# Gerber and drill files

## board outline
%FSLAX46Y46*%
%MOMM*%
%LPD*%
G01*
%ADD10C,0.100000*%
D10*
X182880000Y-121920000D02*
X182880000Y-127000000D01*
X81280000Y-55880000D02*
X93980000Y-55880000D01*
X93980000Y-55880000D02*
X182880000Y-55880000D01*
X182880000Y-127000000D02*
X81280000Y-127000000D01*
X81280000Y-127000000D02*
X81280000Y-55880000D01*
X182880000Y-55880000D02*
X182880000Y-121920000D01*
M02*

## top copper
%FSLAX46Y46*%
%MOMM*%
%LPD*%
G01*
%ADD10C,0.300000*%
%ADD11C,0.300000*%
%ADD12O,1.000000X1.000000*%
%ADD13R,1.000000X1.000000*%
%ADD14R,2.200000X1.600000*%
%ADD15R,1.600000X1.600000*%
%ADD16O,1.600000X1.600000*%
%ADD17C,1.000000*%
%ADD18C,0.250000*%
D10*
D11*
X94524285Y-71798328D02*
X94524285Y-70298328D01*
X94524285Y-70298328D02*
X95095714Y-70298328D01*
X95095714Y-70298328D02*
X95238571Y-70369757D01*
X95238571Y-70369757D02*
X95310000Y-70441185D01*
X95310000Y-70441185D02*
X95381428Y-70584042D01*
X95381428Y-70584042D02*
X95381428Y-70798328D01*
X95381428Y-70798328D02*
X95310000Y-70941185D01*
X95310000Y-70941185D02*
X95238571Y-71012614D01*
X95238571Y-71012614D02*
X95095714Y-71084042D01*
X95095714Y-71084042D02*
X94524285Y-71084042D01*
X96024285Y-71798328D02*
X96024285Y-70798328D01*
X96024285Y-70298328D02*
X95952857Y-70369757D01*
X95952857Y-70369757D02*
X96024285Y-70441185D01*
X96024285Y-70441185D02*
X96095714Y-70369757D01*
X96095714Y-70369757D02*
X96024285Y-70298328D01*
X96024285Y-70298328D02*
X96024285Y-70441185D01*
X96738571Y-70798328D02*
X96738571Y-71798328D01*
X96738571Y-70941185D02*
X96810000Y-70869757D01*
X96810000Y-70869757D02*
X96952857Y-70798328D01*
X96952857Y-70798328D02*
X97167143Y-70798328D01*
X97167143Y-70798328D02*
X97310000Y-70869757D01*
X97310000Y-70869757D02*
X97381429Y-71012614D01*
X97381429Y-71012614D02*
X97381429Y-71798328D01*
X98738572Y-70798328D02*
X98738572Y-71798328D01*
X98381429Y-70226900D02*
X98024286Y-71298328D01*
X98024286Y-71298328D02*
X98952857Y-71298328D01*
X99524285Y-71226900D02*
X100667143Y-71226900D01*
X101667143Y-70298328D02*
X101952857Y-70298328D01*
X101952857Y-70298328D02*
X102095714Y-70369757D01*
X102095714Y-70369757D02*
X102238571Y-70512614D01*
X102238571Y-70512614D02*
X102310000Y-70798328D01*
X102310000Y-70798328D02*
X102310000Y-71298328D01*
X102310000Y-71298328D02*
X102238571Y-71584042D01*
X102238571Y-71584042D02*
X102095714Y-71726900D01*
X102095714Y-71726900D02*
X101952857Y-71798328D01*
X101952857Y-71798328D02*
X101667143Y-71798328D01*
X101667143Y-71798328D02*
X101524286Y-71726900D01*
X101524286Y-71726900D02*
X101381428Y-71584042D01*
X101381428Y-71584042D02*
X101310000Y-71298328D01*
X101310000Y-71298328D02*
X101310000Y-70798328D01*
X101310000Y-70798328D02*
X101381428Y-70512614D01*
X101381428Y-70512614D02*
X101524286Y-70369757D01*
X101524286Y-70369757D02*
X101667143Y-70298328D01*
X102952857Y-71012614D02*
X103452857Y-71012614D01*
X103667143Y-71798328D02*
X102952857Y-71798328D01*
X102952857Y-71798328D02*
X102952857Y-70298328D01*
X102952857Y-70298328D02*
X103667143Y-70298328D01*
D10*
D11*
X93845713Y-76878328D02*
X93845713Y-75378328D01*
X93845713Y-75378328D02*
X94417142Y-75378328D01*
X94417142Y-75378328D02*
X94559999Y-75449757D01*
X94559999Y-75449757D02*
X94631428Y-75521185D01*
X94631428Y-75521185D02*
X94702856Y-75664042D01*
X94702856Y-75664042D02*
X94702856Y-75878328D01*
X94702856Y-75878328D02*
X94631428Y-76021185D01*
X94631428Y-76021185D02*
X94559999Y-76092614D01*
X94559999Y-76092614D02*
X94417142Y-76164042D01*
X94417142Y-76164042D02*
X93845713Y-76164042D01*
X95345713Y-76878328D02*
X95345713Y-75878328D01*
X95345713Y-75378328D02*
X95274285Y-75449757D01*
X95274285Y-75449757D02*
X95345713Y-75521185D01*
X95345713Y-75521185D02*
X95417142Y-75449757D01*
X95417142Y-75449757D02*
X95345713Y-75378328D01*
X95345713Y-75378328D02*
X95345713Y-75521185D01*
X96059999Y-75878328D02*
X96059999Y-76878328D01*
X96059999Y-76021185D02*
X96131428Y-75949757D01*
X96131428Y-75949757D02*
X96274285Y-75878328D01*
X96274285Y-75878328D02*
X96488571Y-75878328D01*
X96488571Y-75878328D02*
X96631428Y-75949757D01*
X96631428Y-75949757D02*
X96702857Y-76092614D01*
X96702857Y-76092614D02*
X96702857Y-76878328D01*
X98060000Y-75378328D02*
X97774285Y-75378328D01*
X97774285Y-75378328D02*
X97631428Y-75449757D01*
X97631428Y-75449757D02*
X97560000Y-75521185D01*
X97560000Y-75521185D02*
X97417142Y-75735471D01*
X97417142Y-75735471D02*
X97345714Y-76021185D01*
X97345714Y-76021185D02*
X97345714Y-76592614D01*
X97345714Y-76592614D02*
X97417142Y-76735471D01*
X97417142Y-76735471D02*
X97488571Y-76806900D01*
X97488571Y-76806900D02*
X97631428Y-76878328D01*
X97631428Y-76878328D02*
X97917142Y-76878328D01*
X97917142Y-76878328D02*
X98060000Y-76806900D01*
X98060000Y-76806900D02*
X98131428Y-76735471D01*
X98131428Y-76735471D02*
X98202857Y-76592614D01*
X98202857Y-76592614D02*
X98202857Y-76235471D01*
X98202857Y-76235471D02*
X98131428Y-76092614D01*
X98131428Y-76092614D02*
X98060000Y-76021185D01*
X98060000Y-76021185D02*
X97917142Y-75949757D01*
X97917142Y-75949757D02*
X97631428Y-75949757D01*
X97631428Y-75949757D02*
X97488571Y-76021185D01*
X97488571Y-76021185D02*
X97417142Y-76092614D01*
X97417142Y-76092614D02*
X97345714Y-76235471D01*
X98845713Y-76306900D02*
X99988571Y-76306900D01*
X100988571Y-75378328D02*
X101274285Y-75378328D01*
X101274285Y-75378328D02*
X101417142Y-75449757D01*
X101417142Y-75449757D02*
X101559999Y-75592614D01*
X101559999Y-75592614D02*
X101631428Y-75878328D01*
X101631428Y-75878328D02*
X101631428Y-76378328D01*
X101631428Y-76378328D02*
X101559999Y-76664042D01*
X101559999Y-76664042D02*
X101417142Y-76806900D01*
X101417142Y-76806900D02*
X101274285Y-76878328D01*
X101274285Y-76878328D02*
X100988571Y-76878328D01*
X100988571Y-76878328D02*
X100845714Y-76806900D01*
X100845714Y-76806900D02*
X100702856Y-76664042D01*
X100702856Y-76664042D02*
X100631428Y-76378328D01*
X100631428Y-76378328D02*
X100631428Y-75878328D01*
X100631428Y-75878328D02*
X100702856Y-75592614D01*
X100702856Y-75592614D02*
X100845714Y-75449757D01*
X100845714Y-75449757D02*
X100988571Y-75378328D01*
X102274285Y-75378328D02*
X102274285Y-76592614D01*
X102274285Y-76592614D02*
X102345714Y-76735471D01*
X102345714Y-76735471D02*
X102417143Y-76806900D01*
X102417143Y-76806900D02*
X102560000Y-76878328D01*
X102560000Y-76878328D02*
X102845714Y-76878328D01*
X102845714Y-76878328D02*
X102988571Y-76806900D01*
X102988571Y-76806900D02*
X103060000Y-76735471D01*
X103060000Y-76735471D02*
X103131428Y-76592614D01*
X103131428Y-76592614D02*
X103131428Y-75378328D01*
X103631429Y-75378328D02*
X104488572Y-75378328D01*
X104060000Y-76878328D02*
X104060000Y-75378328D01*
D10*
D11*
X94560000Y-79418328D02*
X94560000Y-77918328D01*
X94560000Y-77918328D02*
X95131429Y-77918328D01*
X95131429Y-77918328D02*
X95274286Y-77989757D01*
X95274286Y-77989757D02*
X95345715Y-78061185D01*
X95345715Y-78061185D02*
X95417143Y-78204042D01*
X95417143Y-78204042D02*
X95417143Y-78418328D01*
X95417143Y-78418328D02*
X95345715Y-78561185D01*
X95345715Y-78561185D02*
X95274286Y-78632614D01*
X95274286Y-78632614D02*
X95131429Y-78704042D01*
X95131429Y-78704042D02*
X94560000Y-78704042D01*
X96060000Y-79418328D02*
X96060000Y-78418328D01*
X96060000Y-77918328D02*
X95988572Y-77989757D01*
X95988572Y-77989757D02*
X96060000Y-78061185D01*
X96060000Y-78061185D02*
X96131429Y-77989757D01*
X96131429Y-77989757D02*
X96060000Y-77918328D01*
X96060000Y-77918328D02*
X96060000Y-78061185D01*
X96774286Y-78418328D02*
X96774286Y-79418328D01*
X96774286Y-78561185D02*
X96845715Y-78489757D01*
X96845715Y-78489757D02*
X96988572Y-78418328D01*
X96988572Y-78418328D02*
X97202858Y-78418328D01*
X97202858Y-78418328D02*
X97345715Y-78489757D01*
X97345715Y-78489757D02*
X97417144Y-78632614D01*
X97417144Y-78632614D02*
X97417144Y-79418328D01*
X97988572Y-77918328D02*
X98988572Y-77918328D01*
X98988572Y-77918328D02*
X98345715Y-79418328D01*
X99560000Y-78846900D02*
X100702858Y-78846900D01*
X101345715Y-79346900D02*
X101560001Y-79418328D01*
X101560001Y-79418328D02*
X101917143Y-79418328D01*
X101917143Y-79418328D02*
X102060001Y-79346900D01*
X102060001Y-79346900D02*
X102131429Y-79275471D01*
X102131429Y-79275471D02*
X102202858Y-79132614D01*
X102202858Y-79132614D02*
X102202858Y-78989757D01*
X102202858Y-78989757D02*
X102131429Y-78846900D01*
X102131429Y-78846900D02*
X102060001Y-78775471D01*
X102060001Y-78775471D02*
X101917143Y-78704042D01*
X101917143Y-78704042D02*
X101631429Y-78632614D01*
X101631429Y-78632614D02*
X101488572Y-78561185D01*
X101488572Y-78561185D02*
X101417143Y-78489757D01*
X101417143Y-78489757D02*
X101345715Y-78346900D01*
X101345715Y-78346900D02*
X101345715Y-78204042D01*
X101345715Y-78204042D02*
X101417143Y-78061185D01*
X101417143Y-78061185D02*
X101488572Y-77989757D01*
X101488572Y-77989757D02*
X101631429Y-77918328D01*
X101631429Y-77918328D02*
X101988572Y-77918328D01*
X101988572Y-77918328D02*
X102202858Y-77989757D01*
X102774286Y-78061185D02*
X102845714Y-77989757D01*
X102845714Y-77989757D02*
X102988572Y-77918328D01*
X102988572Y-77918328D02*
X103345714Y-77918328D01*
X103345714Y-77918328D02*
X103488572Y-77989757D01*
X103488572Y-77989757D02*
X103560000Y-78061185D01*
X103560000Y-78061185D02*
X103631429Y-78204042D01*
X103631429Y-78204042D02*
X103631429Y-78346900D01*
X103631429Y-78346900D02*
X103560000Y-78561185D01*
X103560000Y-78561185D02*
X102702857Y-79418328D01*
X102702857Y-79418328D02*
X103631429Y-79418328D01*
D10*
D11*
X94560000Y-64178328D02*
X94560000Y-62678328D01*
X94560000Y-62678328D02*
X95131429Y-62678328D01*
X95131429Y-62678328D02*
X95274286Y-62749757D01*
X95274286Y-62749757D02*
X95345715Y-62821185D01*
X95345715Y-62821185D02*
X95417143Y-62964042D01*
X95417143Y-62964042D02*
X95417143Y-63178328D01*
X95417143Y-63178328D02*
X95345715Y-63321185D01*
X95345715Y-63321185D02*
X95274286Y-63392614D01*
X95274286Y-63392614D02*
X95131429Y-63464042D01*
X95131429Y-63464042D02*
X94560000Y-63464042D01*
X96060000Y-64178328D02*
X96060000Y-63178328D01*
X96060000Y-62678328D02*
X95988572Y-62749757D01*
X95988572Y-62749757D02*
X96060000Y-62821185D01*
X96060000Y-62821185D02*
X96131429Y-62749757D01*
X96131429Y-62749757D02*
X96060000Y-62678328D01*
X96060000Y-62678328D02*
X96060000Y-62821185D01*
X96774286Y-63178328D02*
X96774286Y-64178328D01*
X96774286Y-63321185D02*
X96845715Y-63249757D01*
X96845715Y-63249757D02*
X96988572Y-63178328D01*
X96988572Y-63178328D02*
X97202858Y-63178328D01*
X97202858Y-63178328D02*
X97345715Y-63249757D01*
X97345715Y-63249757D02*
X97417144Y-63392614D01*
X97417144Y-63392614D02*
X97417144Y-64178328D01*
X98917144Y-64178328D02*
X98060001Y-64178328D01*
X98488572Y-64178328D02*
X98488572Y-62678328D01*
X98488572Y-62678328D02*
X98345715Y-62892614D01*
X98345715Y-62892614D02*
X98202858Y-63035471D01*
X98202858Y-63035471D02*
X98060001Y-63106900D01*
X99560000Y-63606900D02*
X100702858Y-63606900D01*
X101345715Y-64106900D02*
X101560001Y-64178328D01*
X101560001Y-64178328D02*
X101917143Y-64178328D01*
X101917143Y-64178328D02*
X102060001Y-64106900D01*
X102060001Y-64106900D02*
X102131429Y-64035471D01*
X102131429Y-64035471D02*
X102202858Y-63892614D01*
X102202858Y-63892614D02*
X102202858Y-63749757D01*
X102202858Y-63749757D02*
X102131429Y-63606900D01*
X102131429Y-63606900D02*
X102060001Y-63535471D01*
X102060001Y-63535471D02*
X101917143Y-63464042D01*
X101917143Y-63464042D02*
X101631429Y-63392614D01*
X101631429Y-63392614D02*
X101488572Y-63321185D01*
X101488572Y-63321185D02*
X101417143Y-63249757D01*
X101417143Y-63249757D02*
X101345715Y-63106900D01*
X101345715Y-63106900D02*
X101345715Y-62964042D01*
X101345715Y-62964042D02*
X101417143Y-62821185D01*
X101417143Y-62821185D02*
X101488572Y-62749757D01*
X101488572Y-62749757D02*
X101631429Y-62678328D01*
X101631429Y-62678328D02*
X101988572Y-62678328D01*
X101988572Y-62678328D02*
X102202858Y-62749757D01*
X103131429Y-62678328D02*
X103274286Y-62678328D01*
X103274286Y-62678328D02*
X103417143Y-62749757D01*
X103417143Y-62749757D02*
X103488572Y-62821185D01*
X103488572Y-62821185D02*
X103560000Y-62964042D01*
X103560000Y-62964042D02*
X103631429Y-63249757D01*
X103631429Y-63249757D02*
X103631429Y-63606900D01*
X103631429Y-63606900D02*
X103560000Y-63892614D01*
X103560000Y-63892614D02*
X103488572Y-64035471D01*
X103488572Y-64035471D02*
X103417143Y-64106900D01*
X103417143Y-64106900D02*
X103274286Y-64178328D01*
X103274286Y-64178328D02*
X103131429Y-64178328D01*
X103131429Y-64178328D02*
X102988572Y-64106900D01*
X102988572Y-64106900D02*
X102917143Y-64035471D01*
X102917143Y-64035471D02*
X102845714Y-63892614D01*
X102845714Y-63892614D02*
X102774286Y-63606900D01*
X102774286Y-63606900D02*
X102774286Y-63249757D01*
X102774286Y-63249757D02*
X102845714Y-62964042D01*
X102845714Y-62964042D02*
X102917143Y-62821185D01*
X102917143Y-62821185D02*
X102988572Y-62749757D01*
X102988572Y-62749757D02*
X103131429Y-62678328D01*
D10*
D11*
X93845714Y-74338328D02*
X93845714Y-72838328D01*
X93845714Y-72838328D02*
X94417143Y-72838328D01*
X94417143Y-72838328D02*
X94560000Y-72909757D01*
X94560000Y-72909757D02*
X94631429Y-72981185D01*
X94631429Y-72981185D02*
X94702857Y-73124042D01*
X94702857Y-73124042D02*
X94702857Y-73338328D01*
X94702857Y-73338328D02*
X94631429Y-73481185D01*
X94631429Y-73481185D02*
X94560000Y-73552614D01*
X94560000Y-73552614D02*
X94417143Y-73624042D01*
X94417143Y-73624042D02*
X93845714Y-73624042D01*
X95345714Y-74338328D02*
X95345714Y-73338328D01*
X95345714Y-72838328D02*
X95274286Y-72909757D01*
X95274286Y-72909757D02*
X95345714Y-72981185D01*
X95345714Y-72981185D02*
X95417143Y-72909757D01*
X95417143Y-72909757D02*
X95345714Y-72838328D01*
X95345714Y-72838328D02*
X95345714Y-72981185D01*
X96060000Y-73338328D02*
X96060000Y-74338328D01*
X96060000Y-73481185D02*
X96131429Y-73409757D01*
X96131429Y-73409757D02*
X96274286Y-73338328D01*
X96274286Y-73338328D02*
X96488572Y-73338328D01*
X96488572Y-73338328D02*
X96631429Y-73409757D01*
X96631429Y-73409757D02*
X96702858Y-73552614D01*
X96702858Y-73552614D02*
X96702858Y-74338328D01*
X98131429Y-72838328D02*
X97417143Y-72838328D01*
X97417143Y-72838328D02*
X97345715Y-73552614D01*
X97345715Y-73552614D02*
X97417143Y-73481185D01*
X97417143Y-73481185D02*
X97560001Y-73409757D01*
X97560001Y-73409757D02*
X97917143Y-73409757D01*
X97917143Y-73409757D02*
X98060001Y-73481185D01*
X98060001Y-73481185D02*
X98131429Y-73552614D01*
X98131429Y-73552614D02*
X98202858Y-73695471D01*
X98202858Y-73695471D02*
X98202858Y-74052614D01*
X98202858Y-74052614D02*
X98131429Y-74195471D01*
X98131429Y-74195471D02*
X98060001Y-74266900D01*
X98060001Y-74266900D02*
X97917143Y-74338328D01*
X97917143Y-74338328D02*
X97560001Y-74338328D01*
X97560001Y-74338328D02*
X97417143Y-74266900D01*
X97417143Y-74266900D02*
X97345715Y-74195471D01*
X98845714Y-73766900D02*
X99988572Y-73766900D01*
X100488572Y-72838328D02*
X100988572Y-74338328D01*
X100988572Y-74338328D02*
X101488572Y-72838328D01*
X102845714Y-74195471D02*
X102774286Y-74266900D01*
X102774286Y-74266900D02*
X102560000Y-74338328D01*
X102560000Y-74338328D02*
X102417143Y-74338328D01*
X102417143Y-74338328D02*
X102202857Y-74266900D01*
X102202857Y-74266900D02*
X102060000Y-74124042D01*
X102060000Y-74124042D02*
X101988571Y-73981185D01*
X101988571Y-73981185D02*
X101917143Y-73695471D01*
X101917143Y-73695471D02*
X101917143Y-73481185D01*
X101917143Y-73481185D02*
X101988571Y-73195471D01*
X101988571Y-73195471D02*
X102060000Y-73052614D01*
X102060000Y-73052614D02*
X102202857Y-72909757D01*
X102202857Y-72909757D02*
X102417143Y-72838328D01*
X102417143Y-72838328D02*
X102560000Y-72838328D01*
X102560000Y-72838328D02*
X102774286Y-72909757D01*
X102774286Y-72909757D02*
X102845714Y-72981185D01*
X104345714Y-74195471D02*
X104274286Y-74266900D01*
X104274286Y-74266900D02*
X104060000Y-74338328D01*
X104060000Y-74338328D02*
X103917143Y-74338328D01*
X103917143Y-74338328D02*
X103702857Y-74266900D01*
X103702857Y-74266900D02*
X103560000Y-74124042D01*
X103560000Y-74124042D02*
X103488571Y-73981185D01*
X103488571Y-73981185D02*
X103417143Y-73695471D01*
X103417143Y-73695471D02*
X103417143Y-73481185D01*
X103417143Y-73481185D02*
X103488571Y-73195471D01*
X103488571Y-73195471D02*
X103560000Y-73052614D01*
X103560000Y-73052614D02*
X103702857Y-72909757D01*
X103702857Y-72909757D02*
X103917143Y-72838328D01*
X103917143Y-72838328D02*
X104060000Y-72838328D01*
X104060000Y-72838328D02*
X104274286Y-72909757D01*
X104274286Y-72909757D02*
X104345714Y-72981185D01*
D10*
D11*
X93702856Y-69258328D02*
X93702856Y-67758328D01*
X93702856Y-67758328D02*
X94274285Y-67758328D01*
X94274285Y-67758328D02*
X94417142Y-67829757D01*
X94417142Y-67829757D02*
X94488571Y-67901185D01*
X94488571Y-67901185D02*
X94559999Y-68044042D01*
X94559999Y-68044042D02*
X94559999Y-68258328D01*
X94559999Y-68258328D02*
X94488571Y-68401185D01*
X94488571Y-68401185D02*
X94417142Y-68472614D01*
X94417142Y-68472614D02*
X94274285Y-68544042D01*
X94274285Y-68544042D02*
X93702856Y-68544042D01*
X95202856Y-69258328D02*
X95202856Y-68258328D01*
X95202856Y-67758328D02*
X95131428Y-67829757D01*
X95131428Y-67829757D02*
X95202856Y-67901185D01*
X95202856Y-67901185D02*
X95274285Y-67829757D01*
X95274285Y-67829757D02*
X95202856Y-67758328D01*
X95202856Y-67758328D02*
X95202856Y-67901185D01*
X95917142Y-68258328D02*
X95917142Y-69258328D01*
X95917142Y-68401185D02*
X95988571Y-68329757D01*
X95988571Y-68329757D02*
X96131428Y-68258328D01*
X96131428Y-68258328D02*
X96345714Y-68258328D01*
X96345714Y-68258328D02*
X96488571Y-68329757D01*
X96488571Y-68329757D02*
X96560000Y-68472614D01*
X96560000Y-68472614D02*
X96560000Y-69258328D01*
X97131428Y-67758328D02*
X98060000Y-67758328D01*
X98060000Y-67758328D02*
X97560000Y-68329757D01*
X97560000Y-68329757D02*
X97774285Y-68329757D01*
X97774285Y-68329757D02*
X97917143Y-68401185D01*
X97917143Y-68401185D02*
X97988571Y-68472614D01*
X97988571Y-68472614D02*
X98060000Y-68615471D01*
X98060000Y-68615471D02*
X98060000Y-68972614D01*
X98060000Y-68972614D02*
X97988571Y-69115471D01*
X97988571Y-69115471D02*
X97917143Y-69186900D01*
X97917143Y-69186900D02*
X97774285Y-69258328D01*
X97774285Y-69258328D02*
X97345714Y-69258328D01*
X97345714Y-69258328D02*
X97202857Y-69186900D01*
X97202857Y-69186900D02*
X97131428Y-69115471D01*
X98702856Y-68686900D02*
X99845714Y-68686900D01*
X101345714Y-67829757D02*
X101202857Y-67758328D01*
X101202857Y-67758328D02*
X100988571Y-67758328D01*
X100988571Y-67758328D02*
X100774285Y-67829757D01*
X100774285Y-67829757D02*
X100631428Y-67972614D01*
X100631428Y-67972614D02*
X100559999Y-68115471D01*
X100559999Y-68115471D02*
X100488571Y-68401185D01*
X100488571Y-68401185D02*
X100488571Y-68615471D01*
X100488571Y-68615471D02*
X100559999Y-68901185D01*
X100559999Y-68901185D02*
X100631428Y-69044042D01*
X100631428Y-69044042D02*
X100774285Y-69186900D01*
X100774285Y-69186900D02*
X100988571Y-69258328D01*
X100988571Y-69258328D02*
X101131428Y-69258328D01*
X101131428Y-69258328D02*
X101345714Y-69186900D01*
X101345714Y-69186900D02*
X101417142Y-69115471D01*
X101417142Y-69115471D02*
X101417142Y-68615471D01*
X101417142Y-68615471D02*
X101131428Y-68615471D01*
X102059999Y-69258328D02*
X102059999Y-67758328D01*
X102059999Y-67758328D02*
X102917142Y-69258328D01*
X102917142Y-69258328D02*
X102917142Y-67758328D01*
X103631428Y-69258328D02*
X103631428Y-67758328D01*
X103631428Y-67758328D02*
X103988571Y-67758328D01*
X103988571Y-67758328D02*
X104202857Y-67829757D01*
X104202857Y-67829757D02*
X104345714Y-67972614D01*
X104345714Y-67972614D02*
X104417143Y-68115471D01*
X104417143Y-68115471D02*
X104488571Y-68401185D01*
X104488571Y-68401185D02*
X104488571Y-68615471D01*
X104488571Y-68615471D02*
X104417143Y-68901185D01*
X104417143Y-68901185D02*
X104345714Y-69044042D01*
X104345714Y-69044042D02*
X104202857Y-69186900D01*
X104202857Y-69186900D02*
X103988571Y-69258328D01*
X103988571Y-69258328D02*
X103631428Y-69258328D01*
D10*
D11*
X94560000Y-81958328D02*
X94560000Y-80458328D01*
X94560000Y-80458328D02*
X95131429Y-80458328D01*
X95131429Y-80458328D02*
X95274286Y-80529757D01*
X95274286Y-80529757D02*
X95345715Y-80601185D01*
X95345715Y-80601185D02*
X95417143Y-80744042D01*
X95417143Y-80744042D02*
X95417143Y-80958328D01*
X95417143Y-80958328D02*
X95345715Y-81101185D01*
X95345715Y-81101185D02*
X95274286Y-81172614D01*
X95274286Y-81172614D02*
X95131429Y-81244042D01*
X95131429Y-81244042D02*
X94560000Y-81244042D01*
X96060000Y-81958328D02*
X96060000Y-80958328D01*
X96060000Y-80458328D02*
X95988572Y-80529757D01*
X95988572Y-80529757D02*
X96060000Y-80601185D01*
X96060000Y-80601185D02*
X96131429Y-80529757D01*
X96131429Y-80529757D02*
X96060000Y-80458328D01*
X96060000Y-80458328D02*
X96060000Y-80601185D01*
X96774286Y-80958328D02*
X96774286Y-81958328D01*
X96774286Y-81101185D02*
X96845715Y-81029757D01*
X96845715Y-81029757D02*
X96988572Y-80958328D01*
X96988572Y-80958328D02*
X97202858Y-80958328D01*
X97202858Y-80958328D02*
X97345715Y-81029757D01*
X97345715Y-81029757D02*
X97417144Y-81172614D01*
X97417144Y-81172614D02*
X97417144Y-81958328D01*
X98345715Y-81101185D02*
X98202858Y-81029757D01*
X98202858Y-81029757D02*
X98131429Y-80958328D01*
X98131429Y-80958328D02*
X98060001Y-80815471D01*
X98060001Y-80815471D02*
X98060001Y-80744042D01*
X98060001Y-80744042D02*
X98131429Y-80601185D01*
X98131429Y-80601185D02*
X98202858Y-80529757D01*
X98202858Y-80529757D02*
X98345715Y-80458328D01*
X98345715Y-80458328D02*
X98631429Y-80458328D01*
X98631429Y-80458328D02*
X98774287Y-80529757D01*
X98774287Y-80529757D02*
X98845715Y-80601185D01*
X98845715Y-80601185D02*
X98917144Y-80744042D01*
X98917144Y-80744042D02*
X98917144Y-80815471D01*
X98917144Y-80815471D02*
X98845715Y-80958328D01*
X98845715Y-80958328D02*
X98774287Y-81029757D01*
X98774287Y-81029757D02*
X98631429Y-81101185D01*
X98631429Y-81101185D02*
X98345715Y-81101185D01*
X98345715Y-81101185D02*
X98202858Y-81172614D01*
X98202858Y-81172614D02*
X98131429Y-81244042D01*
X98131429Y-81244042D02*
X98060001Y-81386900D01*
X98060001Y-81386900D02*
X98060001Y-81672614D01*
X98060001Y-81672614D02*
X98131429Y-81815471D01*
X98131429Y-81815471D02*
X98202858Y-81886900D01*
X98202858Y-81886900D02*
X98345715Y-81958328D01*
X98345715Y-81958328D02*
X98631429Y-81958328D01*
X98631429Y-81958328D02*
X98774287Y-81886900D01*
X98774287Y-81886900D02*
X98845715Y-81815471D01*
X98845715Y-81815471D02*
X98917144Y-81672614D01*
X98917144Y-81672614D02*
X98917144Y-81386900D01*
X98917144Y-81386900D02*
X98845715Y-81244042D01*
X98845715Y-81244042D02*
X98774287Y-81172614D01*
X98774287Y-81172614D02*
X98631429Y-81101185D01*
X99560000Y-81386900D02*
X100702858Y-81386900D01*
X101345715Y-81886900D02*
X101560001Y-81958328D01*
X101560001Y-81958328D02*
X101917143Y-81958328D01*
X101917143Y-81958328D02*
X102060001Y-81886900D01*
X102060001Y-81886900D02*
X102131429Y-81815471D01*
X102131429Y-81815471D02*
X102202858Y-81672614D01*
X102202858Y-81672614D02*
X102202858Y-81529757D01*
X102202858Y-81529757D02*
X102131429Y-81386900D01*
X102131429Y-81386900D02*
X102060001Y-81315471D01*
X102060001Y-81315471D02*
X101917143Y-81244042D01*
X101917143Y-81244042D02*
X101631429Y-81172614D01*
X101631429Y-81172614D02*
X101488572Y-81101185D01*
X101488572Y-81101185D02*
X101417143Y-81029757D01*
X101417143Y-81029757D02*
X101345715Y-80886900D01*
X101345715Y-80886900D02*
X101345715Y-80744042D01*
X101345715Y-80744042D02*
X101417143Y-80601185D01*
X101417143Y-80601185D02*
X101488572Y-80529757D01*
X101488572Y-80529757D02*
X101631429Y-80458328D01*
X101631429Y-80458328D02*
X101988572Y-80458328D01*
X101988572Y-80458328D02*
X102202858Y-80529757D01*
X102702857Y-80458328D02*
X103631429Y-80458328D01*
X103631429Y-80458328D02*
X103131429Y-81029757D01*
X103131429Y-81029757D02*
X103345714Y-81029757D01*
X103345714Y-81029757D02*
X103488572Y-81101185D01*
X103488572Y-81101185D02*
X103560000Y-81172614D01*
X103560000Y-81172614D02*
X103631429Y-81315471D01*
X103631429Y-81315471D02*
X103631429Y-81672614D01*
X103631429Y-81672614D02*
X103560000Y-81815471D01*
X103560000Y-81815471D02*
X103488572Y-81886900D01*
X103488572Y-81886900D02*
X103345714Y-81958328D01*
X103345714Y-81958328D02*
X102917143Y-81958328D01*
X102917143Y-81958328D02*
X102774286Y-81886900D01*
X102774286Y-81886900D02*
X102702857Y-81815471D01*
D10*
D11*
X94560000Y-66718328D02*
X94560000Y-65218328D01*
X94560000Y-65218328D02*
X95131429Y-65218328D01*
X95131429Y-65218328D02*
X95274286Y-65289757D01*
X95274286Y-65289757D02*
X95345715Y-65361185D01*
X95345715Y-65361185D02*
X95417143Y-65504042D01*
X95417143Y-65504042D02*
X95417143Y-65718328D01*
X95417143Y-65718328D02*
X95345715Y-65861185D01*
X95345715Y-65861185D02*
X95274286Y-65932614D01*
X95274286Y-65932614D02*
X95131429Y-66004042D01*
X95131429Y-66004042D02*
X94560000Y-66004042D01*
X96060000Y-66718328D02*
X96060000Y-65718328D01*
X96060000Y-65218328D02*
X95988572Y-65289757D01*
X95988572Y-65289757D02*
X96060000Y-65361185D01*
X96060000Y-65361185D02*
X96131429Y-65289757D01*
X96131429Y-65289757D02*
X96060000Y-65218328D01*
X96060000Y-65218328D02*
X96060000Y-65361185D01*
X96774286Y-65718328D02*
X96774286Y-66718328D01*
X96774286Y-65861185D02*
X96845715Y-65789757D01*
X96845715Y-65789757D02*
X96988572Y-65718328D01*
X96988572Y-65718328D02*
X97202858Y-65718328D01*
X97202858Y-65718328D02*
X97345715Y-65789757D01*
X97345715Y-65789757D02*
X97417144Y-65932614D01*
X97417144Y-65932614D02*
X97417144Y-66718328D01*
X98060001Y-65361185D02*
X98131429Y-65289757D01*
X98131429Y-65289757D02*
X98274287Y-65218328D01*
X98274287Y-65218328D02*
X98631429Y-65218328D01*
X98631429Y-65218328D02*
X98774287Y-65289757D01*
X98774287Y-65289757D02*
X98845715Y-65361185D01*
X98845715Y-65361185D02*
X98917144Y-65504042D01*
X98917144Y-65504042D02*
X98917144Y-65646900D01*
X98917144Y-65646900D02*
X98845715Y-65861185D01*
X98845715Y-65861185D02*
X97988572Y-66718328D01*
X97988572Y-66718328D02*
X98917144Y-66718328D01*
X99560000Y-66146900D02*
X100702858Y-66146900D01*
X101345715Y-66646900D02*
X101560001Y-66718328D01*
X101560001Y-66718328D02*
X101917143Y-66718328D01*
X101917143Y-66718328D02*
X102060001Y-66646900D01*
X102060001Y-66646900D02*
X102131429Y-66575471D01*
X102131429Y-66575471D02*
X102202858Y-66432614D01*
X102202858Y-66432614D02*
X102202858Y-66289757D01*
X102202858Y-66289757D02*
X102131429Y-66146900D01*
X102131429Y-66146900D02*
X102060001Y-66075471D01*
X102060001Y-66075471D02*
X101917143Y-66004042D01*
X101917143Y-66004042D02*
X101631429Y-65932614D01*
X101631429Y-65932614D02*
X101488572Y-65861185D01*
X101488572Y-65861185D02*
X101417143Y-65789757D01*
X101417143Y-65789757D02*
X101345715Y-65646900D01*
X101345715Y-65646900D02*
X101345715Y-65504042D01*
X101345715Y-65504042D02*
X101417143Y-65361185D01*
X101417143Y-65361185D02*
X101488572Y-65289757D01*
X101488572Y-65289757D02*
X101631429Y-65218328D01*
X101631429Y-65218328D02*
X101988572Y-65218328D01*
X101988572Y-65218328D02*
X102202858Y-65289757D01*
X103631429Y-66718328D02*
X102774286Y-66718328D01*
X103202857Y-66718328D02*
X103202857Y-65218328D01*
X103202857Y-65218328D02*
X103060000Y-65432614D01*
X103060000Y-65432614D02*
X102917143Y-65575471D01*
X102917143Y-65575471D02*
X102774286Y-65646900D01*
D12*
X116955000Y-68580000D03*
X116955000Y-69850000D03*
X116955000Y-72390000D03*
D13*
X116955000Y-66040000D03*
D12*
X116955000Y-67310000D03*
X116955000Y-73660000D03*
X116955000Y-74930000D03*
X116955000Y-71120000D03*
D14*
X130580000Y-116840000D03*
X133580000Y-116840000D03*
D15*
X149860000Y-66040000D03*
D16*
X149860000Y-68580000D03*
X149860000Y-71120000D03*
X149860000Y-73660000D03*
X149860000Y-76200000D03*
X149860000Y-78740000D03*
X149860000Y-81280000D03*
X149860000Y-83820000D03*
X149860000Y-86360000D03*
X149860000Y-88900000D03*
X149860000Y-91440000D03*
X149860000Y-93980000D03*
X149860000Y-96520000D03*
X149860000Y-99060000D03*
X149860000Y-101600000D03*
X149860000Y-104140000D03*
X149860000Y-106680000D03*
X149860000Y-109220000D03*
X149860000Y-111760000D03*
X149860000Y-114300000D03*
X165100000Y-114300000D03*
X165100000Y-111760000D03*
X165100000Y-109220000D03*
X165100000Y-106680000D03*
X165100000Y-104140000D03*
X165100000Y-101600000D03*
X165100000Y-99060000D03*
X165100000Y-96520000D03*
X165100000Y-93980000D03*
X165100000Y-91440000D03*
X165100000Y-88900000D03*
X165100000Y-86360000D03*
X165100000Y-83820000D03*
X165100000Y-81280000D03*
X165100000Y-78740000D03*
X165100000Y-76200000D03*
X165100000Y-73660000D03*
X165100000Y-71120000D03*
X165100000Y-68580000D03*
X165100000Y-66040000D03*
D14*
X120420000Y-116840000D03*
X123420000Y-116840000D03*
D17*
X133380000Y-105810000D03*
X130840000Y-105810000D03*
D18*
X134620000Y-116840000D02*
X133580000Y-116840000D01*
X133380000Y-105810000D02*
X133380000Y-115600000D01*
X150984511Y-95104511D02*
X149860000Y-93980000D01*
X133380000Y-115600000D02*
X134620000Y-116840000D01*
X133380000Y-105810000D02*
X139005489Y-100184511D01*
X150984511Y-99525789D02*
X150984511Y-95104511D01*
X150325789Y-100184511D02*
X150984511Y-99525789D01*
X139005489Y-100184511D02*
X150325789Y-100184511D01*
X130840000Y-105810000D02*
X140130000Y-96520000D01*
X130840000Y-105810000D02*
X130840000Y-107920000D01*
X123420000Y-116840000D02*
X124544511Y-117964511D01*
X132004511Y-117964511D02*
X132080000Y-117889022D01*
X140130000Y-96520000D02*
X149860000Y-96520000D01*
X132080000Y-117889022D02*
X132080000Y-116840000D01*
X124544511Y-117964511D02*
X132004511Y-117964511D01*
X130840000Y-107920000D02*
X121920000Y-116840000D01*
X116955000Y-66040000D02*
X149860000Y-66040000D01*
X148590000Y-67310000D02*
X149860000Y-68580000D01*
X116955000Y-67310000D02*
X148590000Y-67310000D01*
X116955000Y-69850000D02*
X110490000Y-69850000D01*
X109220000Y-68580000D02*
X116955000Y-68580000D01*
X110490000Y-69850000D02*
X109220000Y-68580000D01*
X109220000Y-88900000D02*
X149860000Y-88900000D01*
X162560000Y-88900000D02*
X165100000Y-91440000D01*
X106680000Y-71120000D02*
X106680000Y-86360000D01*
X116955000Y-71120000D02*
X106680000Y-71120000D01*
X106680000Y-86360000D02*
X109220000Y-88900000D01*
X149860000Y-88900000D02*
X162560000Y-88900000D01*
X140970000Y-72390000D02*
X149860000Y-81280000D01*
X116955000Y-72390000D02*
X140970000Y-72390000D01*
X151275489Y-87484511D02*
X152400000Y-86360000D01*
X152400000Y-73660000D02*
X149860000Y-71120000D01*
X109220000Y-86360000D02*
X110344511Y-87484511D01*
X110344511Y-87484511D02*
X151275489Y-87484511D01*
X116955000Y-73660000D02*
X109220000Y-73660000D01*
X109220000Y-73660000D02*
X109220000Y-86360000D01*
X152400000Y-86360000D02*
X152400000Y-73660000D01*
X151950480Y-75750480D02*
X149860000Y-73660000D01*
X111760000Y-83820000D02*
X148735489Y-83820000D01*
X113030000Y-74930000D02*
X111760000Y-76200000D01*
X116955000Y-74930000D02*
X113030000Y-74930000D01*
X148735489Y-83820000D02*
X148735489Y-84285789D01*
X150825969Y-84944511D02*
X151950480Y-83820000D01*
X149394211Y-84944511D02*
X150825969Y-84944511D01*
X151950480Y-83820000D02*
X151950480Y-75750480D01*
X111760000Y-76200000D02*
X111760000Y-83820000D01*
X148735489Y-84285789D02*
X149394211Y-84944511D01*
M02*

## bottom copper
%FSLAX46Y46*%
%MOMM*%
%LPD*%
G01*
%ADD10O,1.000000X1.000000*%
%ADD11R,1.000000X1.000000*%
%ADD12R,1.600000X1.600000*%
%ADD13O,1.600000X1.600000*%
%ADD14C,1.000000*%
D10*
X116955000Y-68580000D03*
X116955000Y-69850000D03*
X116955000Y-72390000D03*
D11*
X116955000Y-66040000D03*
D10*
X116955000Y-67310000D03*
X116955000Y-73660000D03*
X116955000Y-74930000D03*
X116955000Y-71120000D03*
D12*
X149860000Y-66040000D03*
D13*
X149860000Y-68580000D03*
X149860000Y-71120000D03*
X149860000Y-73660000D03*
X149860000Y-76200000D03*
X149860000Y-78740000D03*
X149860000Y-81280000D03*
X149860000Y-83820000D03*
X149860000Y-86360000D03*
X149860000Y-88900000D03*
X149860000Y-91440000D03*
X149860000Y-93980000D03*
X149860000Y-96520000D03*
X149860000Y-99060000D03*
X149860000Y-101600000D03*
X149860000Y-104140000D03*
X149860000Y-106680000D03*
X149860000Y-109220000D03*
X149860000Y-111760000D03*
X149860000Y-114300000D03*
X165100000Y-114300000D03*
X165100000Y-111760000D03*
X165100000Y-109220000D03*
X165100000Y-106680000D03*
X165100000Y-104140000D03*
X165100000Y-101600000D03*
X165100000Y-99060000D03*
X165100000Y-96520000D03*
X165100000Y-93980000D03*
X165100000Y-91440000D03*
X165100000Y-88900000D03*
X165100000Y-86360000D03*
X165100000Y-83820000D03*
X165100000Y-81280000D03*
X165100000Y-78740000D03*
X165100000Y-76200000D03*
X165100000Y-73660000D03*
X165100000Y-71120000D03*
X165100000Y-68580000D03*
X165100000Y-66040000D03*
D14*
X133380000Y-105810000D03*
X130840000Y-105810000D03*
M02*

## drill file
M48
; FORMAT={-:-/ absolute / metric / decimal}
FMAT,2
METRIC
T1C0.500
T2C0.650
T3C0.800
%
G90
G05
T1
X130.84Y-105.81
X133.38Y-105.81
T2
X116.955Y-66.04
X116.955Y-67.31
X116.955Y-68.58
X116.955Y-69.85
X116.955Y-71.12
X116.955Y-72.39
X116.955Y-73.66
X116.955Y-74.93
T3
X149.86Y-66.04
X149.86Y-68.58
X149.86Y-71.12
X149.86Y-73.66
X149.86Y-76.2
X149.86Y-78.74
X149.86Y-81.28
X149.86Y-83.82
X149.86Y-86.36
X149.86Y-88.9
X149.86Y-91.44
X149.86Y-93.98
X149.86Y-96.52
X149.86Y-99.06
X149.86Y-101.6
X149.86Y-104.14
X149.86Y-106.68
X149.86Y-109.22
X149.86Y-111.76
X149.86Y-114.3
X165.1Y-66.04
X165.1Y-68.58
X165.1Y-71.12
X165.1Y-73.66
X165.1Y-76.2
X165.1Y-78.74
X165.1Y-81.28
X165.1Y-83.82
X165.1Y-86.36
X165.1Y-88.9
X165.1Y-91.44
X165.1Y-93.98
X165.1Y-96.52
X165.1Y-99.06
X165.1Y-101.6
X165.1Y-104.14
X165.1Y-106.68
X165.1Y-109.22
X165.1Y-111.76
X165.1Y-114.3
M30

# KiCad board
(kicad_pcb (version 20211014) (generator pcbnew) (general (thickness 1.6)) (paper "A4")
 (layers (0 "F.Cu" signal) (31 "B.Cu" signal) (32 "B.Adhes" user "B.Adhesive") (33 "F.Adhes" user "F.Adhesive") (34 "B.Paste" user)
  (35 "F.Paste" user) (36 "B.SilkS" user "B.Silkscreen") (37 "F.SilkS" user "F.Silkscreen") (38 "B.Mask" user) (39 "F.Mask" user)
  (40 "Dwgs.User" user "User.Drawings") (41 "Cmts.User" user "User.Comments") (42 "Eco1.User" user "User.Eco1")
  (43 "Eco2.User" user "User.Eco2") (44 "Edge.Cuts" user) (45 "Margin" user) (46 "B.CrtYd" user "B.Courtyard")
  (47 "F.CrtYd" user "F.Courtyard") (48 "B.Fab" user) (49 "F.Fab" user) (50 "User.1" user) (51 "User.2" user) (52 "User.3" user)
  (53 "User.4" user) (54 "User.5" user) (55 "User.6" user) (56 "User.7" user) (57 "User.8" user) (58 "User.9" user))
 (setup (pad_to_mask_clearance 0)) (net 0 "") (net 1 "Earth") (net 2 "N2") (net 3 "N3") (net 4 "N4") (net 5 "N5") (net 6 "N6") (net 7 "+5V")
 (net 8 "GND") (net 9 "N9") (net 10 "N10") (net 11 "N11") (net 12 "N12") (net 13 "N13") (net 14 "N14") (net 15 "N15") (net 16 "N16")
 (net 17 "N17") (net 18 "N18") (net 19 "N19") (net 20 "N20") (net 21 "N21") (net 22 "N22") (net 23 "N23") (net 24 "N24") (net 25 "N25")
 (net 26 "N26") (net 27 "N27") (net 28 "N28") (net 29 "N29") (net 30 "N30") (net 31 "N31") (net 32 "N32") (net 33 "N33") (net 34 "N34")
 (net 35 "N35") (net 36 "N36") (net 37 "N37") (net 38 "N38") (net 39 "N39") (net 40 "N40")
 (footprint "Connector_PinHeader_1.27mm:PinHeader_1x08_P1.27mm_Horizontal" (layer "F.Cu") (at 116.955 66.04)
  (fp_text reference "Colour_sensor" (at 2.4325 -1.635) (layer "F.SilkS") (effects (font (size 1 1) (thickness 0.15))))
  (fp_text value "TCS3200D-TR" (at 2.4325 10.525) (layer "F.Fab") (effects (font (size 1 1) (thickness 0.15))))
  (pad "GND" thru_hole oval (at 0 2.54) (size 1 1) (drill 0.65) (layers *.Cu *.Mask) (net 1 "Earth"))
  (pad "OE" thru_hole oval (at 0 3.81) (size 1 1) (drill 0.65) (layers *.Cu *.Mask) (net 1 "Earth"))
  (pad "OUT" thru_hole oval (at 0 6.35) (size 1 1) (drill 0.65) (layers *.Cu *.Mask) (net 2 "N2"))
  (pad "S0" thru_hole rect (at 0 0) (size 1 1) (drill 0.65) (layers *.Cu *.Mask) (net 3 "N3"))
  (pad "S1" thru_hole oval (at 0 1.27) (size 1 1) (drill 0.65) (layers *.Cu *.Mask) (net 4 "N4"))
  (pad "S2" thru_hole oval (at 0 7.62) (size 1 1) (drill 0.65) (layers *.Cu *.Mask) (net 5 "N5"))
  (pad "S3" thru_hole oval (at 0 8.89) (size 1 1) (drill 0.65) (layers *.Cu *.Mask) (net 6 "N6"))
  (pad "VCC" thru_hole oval (at 0 5.08) (size 1 1) (drill 0.65) (layers *.Cu *.Mask) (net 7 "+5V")))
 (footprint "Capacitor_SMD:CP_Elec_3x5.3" (layer "F.Cu") (at 132.08 116.84)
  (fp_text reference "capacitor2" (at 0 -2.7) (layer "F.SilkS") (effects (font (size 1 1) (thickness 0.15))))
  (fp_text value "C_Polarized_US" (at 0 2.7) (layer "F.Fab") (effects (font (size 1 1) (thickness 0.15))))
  (pad "1" smd rect (at -1.5 0) (size 2.2 1.6) (layers "F.Cu" "F.Paste" "F.Mask") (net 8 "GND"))
  (pad "2" smd rect (at 1.5 0) (size 2.2 1.6) (layers "F.Cu" "F.Paste" "F.Mask") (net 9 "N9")))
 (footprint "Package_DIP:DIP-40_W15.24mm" (layer "F.Cu") (at 149.86 66.04)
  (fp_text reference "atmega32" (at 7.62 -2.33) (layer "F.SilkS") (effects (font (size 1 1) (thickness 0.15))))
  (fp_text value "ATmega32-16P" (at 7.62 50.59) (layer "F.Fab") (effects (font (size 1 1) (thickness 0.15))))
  (pad "1" thru_hole rect (at 0 0) (size 1.6 1.6) (drill 0.8) (layers *.Cu *.Mask) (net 3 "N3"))
  (pad "2" thru_hole oval (at 0 2.54) (size 1.6 1.6) (drill 0.8) (layers *.Cu *.Mask) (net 4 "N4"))
  (pad "3" thru_hole oval (at 0 5.08) (size 1.6 1.6) (drill 0.8) (layers *.Cu *.Mask) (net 5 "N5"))
  (pad "4" thru_hole oval (at 0 7.62) (size 1.6 1.6) (drill 0.8) (layers *.Cu *.Mask) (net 6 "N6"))
  (pad "5" thru_hole oval (at 0 10.16) (size 1.6 1.6) (drill 0.8) (layers *.Cu *.Mask) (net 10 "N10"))
  (pad "6" thru_hole oval (at 0 12.7) (size 1.6 1.6) (drill 0.8) (layers *.Cu *.Mask) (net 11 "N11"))
  (pad "7" thru_hole oval (at 0 15.24) (size 1.6 1.6) (drill 0.8) (layers *.Cu *.Mask) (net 2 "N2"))
  (pad "8" thru_hole oval (at 0 17.78) (size 1.6 1.6) (drill 0.8) (layers *.Cu *.Mask) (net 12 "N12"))
  (pad "9" thru_hole oval (at 0 20.32) (size 1.6 1.6) (drill 0.8) (layers *.Cu *.Mask) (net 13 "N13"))
  (pad "10" thru_hole oval (at 0 22.86) (size 1.6 1.6) (drill 0.8) (layers *.Cu *.Mask) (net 7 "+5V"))
  (pad "11" thru_hole oval (at 0 25.4) (size 1.6 1.6) (drill 0.8) (layers *.Cu *.Mask) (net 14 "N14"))
  (pad "12" thru_hole oval (at 0 27.94) (size 1.6 1.6) (drill 0.8) (layers *.Cu *.Mask) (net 9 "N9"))
  (pad "13" thru_hole oval (at 0 30.48) (size 1.6 1.6) (drill 0.8) (layers *.Cu *.Mask) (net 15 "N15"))
  (pad "14" thru_hole oval (at 0 33.02) (size 1.6 1.6) (drill 0.8) (layers *.Cu *.Mask) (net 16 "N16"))
  (pad "15" thru_hole oval (at 0 35.56) (size 1.6 1.6) (drill 0.8) (layers *.Cu *.Mask) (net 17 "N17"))
  (pad "16" thru_hole oval (at 0 38.1) (size 1.6 1.6) (drill 0.8) (layers *.Cu *.Mask) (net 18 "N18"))
  (pad "17" thru_hole oval (at 0 40.64) (size 1.6 1.6) (drill 0.8) (layers *.Cu *.Mask) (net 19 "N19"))
  (pad "18" thru_hole oval (at 0 43.18) (size 1.6 1.6) (drill 0.8) (layers *.Cu *.Mask) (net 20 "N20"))
  (pad "19" thru_hole oval (at 0 45.72) (size 1.6 1.6) (drill 0.8) (layers *.Cu *.Mask) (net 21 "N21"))
  (pad "20" thru_hole oval (at 0 48.26) (size 1.6 1.6) (drill 0.8) (layers *.Cu *.Mask) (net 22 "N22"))
  (pad "21" thru_hole oval (at 15.24 48.26) (size 1.6 1.6) (drill 0.8) (layers *.Cu *.Mask) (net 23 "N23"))
  (pad "22" thru_hole oval (at 15.24 45.72) (size 1.6 1.6) (drill 0.8) (layers *.Cu *.Mask) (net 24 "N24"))
  (pad "23" thru_hole oval (at 15.24 43.18) (size 1.6 1.6) (drill 0.8) (layers *.Cu *.Mask) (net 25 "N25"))
  (pad "24" thru_hole oval (at 15.24 40.64) (size 1.6 1.6) (drill 0.8) (layers *.Cu *.Mask) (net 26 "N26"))
  (pad "25" thru_hole oval (at 15.24 38.1) (size 1.6 1.6) (drill 0.8) (layers *.Cu *.Mask) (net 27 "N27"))
  (pad "26" thru_hole oval (at 15.24 35.56) (size 1.6 1.6) (drill 0.8) (layers *.Cu *.Mask) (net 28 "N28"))
  (pad "27" thru_hole oval (at 15.24 33.02) (size 1.6 1.6) (drill 0.8) (layers *.Cu *.Mask) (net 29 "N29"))
  (pad "28" thru_hole oval (at 15.24 30.48) (size 1.6 1.6) (drill 0.8) (layers *.Cu *.Mask) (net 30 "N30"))
  (pad "29" thru_hole oval (at 15.24 27.94) (size 1.6 1.6) (drill 0.8) (layers *.Cu *.Mask) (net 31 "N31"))
  (pad "30" thru_hole oval (at 15.24 25.4) (size 1.6 1.6) (drill 0.8) (layers *.Cu *.Mask) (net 7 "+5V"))
  (pad "31" thru_hole oval (at 15.24 22.86) (size 1.6 1.6) (drill 0.8) (layers *.Cu *.Mask) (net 14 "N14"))
  (pad "32" thru_hole oval (at 15.24 20.32) (size 1.6 1.6) (drill 0.8) (layers *.Cu *.Mask) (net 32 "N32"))
  (pad "33" thru_hole oval (at 15.24 17.78) (size 1.6 1.6) (drill 0.8) (layers *.Cu *.Mask) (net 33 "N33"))
  (pad "34" thru_hole oval (at 15.24 15.24) (size 1.6 1.6) (drill 0.8) (layers *.Cu *.Mask) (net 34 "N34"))
  (pad "35" thru_hole oval (at 15.24 12.7) (size 1.6 1.6) (drill 0.8) (layers *.Cu *.Mask) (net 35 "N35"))
  (pad "36" thru_hole oval (at 15.24 10.16) (size 1.6 1.6) (drill 0.8) (layers *.Cu *.Mask) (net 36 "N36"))
  (pad "37" thru_hole oval (at 15.24 7.62) (size 1.6 1.6) (drill 0.8) (layers *.Cu *.Mask) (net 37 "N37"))
  (pad "38" thru_hole oval (at 15.24 5.08) (size 1.6 1.6) (drill 0.8) (layers *.Cu *.Mask) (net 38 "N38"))
  (pad "39" thru_hole oval (at 15.24 2.54) (size 1.6 1.6) (drill 0.8) (layers *.Cu *.Mask) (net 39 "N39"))
  (pad "40" thru_hole oval (at 15.24 0) (size 1.6 1.6) (drill 0.8) (layers *.Cu *.Mask) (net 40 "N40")))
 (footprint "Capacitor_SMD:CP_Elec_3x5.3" (layer "F.Cu") (at 121.92 116.84)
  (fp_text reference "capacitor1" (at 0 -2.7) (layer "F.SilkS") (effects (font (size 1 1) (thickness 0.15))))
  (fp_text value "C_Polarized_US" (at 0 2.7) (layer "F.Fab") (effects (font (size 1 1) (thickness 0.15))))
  (pad "1" smd rect (at -1.5 0) (size 2.2 1.6) (layers "F.Cu" "F.Paste" "F.Mask") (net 8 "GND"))
  (pad "2" smd rect (at 1.5 0) (size 2.2 1.6) (layers "F.Cu" "F.Paste" "F.Mask") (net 15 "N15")))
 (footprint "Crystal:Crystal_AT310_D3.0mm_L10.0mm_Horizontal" (layer "F.Cu") (at 133.38 105.81 180)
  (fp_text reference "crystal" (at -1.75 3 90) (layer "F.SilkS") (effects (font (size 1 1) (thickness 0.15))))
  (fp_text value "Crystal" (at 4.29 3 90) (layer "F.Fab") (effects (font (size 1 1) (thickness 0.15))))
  (pad "1" thru_hole circle (at 0 0 180) (size 1 1) (drill 0.5) (layers *.Cu *.Mask) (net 9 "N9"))
  (pad "2" thru_hole circle (at 2.54 0 180) (size 1 1) (drill 0.5) (layers *.Cu *.Mask) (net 15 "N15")))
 (gr_line (start 182.88 121.92) (end 182.88 127) (layer "Edge.Cuts") (width 0.1))
 (gr_line (start 81.28 55.88) (end 93.98 55.88) (layer "Edge.Cuts") (width 0.1))
 (gr_line (start 93.98 55.88) (end 182.88 55.88) (layer "Edge.Cuts") (width 0.1))
 (gr_line (start 182.88 127) (end 81.28 127) (layer "Edge.Cuts") (width 0.1))
 (gr_line (start 81.28 127) (end 81.28 55.88) (layer "Edge.Cuts") (width 0.1))
 (gr_line (start 182.88 55.88) (end 182.88 121.92) (layer "Edge.Cuts") (width 0.1))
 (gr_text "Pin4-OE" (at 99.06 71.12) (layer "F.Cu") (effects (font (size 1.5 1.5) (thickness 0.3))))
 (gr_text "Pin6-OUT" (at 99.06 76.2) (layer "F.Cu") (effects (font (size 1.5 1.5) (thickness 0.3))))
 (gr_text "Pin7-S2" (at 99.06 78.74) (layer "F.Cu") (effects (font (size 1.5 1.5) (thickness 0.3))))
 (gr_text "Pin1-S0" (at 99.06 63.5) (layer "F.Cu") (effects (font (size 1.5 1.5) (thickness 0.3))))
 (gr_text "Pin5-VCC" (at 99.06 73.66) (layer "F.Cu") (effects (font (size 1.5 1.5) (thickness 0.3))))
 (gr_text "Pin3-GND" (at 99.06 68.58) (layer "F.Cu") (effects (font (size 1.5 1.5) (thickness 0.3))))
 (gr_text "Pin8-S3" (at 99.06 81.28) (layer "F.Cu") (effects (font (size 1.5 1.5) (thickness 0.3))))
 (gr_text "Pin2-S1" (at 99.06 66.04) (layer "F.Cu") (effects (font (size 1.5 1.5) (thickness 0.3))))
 (segment (start 134.62 116.84) (end 133.58 116.84) (width 0.25) (layer "F.Cu") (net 9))
 (segment (start 133.38 105.81) (end 133.38 115.6) (width 0.25) (layer "F.Cu") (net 9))
 (segment (start 150.984511 95.104511) (end 149.86 93.98) (width 0.25) (layer "F.Cu") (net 9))
 (segment (start 133.38 115.6) (end 134.62 116.84) (width 0.25) (layer "F.Cu") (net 9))
 (segment (start 133.38 105.81) (end 139.005489 100.184511) (width 0.25) (layer "F.Cu") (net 9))
 (segment (start 150.984511 99.525789) (end 150.984511 95.104511) (width 0.25) (layer "F.Cu") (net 9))
 (segment (start 150.325789 100.184511) (end 150.984511 99.525789) (width 0.25) (layer "F.Cu") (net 9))
 (segment (start 139.005489 100.184511) (end 150.325789 100.184511) (width 0.25) (layer "F.Cu") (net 9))
 (segment (start 130.84 105.81) (end 140.13 96.52) (width 0.25) (layer "F.Cu") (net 15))
 (segment (start 130.84 105.81) (end 130.84 107.92) (width 0.25) (layer "F.Cu") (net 15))
 (segment (start 123.42 116.84) (end 124.544511 117.964511) (width 0.25) (layer "F.Cu") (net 15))
 (segment (start 132.004511 117.964511) (end 132.08 117.889022) (width 0.25) (layer "F.Cu") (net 15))
 (segment (start 140.13 96.52) (end 149.86 96.52) (width 0.25) (layer "F.Cu") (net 15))
 (segment (start 132.08 117.889022) (end 132.08 116.84) (width 0.25) (layer "F.Cu") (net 15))
 (segment (start 124.544511 117.964511) (end 132.004511 117.964511) (width 0.25) (layer "F.Cu") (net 15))
 (segment (start 130.84 107.92) (end 121.92 116.84) (width 0.25) (layer "F.Cu") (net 15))
 (segment (start 116.955 66.04) (end 149.86 66.04) (width 0.25) (layer "F.Cu") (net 3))
 (segment (start 148.59 67.31) (end 149.86 68.58) (width 0.25) (layer "F.Cu") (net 4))
 (segment (start 116.955 67.31) (end 148.59 67.31) (width 0.25) (layer "F.Cu") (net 4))
 (segment (start 116.955 69.85) (end 110.49 69.85) (width 0.25) (layer "F.Cu") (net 1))
 (segment (start 109.22 68.58) (end 116.955 68.58) (width 0.25) (layer "F.Cu") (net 1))
 (segment (start 110.49 69.85) (end 109.22 68.58) (width 0.25) (layer "F.Cu") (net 1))
 (segment (start 109.22 88.9) (end 149.86 88.9) (width 0.25) (layer "F.Cu") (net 7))
 (segment (start 162.56 88.9) (end 165.1 91.44) (width 0.25) (layer "F.Cu") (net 7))
 (segment (start 106.68 71.12) (end 106.68 86.36) (width 0.25) (layer "F.Cu") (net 7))
 (segment (start 116.955 71.12) (end 106.68 71.12) (width 0.25) (layer "F.Cu") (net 7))
 (segment (start 106.68 86.36) (end 109.22 88.9) (width 0.25) (layer "F.Cu") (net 7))
 (segment (start 149.86 88.9) (end 162.56 88.9) (width 0.25) (layer "F.Cu") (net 7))
 (segment (start 140.97 72.39) (end 149.86 81.28) (width 0.25) (layer "F.Cu") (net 2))
 (segment (start 116.955 72.39) (end 140.97 72.39) (width 0.25) (layer "F.Cu") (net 2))
 (segment (start 151.275489 87.484511) (end 152.4 86.36) (width 0.25) (layer "F.Cu") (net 5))
 (segment (start 152.4 73.66) (end 149.86 71.12) (width 0.25) (layer "F.Cu") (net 5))
 (segment (start 109.22 86.36) (end 110.344511 87.484511) (width 0.25) (layer "F.Cu") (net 5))
 (segment (start 110.344511 87.484511) (end 151.275489 87.484511) (width 0.25) (layer "F.Cu") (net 5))
 (segment (start 116.955 73.66) (end 109.22 73.66) (width 0.25) (layer "F.Cu") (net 5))
 (segment (start 109.22 73.66) (end 109.22 86.36) (width 0.25) (layer "F.Cu") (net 5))
 (segment (start 152.4 86.36) (end 152.4 73.66) (width 0.25) (layer "F.Cu") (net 5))
 (segment (start 151.95048 75.75048) (end 149.86 73.66) (width 0.25) (layer "F.Cu") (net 6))
 (segment (start 111.76 83.82) (end 148.735489 83.82) (width 0.25) (layer "F.Cu") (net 6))
 (segment (start 113.03 74.93) (end 111.76 76.2) (width 0.25) (layer "F.Cu") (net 6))
 (segment (start 116.955 74.93) (end 113.03 74.93) (width 0.25) (layer "F.Cu") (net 6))
 (segment (start 148.735489 83.82) (end 148.735489 84.285789) (width 0.25) (layer "F.Cu") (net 6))
 (segment (start 150.825969 84.944511) (end 151.95048 83.82) (width 0.25) (layer "F.Cu") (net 6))
 (segment (start 149.394211 84.944511) (end 150.825969 84.944511) (width 0.25) (layer "F.Cu") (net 6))
 (segment (start 151.95048 83.82) (end 151.95048 75.75048) (width 0.25) (layer "F.Cu") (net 6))
 (segment (start 111.76 76.2) (end 111.76 83.82) (width 0.25) (layer "F.Cu") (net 6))
 (segment (start 148.735489 84.285789) (end 149.394211 84.944511) (width 0.25) (layer "F.Cu") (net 6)))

